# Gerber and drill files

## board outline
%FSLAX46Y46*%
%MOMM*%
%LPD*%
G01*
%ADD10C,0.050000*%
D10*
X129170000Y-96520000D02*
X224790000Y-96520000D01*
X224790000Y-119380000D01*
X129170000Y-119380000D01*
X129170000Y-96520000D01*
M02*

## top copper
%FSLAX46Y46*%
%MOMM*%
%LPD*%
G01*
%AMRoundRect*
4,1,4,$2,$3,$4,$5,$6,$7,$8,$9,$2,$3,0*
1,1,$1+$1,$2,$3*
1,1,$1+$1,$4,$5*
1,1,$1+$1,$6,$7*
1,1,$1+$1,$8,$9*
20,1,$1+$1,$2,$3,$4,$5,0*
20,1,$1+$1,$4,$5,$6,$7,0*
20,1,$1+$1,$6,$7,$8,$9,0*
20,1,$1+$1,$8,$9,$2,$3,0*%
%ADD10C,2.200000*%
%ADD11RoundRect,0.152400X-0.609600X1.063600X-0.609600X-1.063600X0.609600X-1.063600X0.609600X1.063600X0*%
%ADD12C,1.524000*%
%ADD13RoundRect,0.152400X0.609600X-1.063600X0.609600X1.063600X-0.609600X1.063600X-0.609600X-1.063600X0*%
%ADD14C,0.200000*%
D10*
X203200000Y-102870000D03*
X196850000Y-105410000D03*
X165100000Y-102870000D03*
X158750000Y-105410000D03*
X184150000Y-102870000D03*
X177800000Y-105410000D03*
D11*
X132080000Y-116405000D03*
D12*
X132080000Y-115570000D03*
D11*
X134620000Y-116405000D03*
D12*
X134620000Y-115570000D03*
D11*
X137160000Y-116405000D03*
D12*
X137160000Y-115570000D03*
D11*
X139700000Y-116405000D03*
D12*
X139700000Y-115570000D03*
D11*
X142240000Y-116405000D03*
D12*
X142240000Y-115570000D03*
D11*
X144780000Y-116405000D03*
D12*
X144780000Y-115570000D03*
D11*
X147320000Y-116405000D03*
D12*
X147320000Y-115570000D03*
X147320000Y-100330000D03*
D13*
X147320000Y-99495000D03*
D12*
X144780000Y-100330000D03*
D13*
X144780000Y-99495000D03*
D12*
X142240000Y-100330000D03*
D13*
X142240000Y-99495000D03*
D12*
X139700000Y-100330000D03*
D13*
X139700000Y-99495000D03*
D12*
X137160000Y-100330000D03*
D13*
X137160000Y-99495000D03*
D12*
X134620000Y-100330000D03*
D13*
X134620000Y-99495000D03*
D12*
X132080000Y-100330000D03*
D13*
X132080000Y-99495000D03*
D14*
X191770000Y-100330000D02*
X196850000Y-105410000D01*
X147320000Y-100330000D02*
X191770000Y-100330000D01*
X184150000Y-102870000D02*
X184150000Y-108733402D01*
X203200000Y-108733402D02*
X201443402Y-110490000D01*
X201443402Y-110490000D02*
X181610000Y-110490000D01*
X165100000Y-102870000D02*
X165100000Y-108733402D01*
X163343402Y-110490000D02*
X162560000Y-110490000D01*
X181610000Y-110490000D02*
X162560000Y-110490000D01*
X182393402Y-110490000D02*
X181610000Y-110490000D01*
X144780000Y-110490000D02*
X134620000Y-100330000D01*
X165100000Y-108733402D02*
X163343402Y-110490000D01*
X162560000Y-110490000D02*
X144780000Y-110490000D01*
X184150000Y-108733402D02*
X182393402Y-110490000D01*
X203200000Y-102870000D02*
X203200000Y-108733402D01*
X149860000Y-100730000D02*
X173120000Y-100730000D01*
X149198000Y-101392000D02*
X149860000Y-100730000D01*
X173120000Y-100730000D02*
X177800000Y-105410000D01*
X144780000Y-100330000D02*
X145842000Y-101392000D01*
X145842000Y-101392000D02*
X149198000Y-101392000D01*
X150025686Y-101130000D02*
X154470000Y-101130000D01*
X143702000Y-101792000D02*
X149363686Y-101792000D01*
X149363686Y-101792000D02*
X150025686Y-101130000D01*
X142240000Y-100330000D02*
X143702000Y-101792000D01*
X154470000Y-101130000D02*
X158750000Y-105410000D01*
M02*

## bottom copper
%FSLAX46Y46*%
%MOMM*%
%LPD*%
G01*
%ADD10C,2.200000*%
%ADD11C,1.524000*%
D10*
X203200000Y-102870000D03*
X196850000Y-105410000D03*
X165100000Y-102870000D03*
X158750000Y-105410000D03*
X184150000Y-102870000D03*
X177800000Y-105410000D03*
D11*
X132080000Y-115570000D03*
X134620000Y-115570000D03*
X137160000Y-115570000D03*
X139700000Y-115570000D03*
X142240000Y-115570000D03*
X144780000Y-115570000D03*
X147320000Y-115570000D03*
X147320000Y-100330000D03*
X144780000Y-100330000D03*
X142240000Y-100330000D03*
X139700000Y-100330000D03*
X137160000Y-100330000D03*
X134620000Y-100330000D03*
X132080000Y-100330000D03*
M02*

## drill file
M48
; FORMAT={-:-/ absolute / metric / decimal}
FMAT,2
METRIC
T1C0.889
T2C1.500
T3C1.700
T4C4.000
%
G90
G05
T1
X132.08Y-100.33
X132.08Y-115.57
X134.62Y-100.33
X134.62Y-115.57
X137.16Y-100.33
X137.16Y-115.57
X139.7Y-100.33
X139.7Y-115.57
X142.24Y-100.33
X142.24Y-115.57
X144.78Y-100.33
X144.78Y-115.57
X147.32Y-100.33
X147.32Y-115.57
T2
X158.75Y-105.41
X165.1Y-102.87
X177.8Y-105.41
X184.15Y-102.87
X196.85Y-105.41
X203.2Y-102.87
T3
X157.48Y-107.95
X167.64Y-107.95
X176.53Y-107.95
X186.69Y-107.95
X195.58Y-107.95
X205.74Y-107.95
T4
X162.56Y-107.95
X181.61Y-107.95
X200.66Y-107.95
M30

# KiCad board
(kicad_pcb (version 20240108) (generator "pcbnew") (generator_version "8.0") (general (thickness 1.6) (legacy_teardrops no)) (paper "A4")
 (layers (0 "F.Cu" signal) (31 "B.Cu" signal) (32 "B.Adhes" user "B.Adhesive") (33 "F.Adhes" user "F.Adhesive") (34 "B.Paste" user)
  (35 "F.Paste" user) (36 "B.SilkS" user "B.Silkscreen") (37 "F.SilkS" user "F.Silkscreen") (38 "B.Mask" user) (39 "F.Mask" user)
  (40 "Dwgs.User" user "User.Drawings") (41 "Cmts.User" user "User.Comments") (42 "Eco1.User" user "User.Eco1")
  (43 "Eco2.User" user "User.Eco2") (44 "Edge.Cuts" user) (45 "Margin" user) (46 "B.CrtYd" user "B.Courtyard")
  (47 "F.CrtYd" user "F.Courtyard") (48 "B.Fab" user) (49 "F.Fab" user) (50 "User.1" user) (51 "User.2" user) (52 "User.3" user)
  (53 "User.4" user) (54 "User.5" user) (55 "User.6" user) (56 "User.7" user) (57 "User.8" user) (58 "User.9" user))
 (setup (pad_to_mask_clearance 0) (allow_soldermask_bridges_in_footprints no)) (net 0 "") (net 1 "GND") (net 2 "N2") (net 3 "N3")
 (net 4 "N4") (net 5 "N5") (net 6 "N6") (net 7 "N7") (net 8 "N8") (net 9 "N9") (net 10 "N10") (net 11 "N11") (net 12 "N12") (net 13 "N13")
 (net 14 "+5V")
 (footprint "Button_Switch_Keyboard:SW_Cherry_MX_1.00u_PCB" (layer "F.Cu") (at 203.2 102.87)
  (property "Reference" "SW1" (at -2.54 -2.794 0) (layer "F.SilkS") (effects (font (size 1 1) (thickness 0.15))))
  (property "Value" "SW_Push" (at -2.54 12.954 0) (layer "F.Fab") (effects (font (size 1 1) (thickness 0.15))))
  (pad "" np_thru_hole circle (at -7.62 5.08) (size 1.7 1.7) (drill 1.7) (layers "*.Cu" "*.Mask"))
  (pad "" np_thru_hole circle (at -2.54 5.08) (size 4 4) (drill 4) (layers "*.Cu" "*.Mask"))
  (pad "" np_thru_hole circle (at 2.54 5.08) (size 1.7 1.7) (drill 1.7) (layers "*.Cu" "*.Mask"))
  (pad "1" thru_hole circle (at 0 0) (size 2.2 2.2) (drill 1.5) (layers "*.Cu" "*.Mask") (remove_unused_layers no) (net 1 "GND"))
  (pad "2" thru_hole circle (at -6.35 2.54) (size 2.2 2.2) (drill 1.5) (layers "*.Cu" "*.Mask") (remove_unused_layers no) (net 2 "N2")))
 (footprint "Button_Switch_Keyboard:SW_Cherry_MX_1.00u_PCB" (layer "F.Cu") (at 165.1 102.87)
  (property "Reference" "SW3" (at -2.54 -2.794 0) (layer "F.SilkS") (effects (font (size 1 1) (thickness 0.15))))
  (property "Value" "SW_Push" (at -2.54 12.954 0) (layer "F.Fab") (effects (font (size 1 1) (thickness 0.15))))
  (pad "" np_thru_hole circle (at -7.62 5.08) (size 1.7 1.7) (drill 1.7) (layers "*.Cu" "*.Mask"))
  (pad "" np_thru_hole circle (at -2.54 5.08) (size 4 4) (drill 4) (layers "*.Cu" "*.Mask"))
  (pad "" np_thru_hole circle (at 2.54 5.08) (size 1.7 1.7) (drill 1.7) (layers "*.Cu" "*.Mask"))
  (pad "1" thru_hole circle (at 0 0) (size 2.2 2.2) (drill 1.5) (layers "*.Cu" "*.Mask") (remove_unused_layers no) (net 1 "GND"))
  (pad "2" thru_hole circle (at -6.35 2.54) (size 2.2 2.2) (drill 1.5) (layers "*.Cu" "*.Mask") (remove_unused_layers no) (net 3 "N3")))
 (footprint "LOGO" (layer "F.Cu") (at 214.63 100.33)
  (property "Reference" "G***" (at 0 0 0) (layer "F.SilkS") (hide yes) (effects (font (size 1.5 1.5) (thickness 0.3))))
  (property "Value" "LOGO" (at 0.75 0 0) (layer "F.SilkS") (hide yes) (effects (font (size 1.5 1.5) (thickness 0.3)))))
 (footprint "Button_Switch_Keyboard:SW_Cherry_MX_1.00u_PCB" (layer "F.Cu") (at 184.15 102.87)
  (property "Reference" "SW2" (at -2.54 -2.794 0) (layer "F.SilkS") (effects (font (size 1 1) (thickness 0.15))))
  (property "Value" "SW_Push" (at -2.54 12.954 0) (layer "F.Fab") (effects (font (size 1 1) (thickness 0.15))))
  (pad "" np_thru_hole circle (at -7.62 5.08) (size 1.7 1.7) (drill 1.7) (layers "*.Cu" "*.Mask"))
  (pad "" np_thru_hole circle (at -2.54 5.08) (size 4 4) (drill 4) (layers "*.Cu" "*.Mask"))
  (pad "" np_thru_hole circle (at 2.54 5.08) (size 1.7 1.7) (drill 1.7) (layers "*.Cu" "*.Mask"))
  (pad "1" thru_hole circle (at 0 0) (size 2.2 2.2) (drill 1.5) (layers "*.Cu" "*.Mask") (remove_unused_layers no) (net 1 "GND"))
  (pad "2" thru_hole circle (at -6.35 2.54) (size 2.2 2.2) (drill 1.5) (layers "*.Cu" "*.Mask") (remove_unused_layers no) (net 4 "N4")))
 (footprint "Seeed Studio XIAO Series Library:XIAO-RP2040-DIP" (layer "F.Cu") (at 139.7 107.95 90)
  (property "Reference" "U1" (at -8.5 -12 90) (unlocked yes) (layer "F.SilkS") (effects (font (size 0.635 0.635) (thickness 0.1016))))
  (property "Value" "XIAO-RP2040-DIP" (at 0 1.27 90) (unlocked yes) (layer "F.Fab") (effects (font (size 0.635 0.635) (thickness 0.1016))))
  (pad "1" smd roundrect (at -8.455 -7.62 270) (size 2.432 1.524) (layers "F.Cu" "F.Mask") (roundrect_rratio 0.1) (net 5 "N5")
   (thermal_bridge_angle 45))
  (pad "1" thru_hole circle (at -7.62 -7.62 270) (size 1.524 1.524) (drill 0.889) (layers "*.Cu" "*.Mask") (remove_unused_layers no)
   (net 5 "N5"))
  (pad "2" smd roundrect (at -8.455 -5.08 270) (size 2.432 1.524) (layers "F.Cu" "F.Mask") (roundrect_rratio 0.1) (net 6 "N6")
   (thermal_bridge_angle 45))
  (pad "2" thru_hole circle (at -7.62 -5.08 270) (size 1.524 1.524) (drill 0.889) (layers "*.Cu" "*.Mask") (remove_unused_layers no)
   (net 6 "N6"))
  (pad "3" smd roundrect (at -8.455 -2.54 270) (size 2.432 1.524) (layers "F.Cu" "F.Mask") (roundrect_rratio 0.1) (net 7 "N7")
   (thermal_bridge_angle 45))
  (pad "3" thru_hole circle (at -7.62 -2.54 270) (size 1.524 1.524) (drill 0.889) (layers "*.Cu" "*.Mask") (remove_unused_layers no)
   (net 7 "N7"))
  (pad "4" smd roundrect (at -8.455 0 270) (size 2.432 1.524) (layers "F.Cu" "F.Mask") (roundrect_rratio 0.1) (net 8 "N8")
   (thermal_bridge_angle 45))
  (pad "4" thru_hole circle (at -7.62 0 270) (size 1.524 1.524) (drill 0.889) (layers "*.Cu" "*.Mask") (remove_unused_layers no)
   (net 8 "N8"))
  (pad "5" smd roundrect (at -8.455 2.54 270) (size 2.432 1.524) (layers "F.Cu" "F.Mask") (roundrect_rratio 0.1) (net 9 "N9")
   (thermal_bridge_angle 45))
  (pad "5" thru_hole circle (at -7.62 2.54 270) (size 1.524 1.524) (drill 0.889) (layers "*.Cu" "*.Mask") (remove_unused_layers no)
   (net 9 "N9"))
  (pad "6" smd roundrect (at -8.455 5.08 270) (size 2.432 1.524) (layers "F.Cu" "F.Mask") (roundrect_rratio 0.1) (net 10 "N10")
   (thermal_bridge_angle 45))
  (pad "6" thru_hole circle (at -7.62 5.08 270) (size 1.524 1.524) (drill 0.889) (layers "*.Cu" "*.Mask") (remove_unused_layers no)
   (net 10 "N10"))
  (pad "7" smd roundrect (at -8.455 7.62 270) (size 2.432 1.524) (layers "F.Cu" "F.Mask") (roundrect_rratio 0.1) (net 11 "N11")
   (thermal_bridge_angle 45))
  (pad "7" thru_hole circle (at -7.62 7.62 270) (size 1.524 1.524) (drill 0.889) (layers "*.Cu" "*.Mask") (remove_unused_layers no)
   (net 11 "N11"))
  (pad "8" thru_hole circle (at 7.62 7.62 90) (size 1.524 1.524) (drill 0.889) (layers "*.Cu" "*.Mask") (remove_unused_layers no)
   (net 2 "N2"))
  (pad "8" smd roundrect (at 8.455 7.62 90) (size 2.432 1.524) (layers "F.Cu" "F.Mask") (roundrect_rratio 0.1) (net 2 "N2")
   (thermal_bridge_angle 45))
  (pad "9" thru_hole circle (at 7.62 5.08 90) (size 1.524 1.524) (drill 0.889) (layers "*.Cu" "*.Mask") (remove_unused_layers no)
   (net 4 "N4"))
  (pad "9" smd roundrect (at 8.455 5.08 90) (size 2.432 1.524) (layers "F.Cu" "F.Mask") (roundrect_rratio 0.1) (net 4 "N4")
   (thermal_bridge_angle 45))
  (pad "10" thru_hole circle (at 7.62 2.54 90) (size 1.524 1.524) (drill 0.889) (layers "*.Cu" "*.Mask") (remove_unused_layers no)
   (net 3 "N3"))
  (pad "10" smd roundrect (at 8.455 2.54 90) (size 2.432 1.524) (layers "F.Cu" "F.Mask") (roundrect_rratio 0.1) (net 3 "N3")
   (thermal_bridge_angle 45))
  (pad "11" thru_hole circle (at 7.62 0 90) (size 1.524 1.524) (drill 0.889) (layers "*.Cu" "*.Mask") (remove_unused_layers no)
   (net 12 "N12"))
  (pad "11" smd roundrect (at 8.455 0 90) (size 2.432 1.524) (layers "F.Cu" "F.Mask") (roundrect_rratio 0.1) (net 12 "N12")
   (thermal_bridge_angle 45))
  (pad "12" thru_hole circle (at 7.62 -2.54 90) (size 1.524 1.524) (drill 0.889) (layers "*.Cu" "*.Mask") (remove_unused_layers no)
   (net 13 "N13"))
  (pad "12" smd roundrect (at 8.455 -2.54 90) (size 2.432 1.524) (layers "F.Cu" "F.Mask") (roundrect_rratio 0.1) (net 13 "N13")
   (thermal_bridge_angle 45))
  (pad "13" thru_hole circle (at 7.62 -5.08 90) (size 1.524 1.524) (drill 0.889) (layers "*.Cu" "*.Mask") (remove_unused_layers no)
   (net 1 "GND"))
  (pad "13" smd roundrect (at 8.455 -5.08 90) (size 2.432 1.524) (layers "F.Cu" "F.Mask") (roundrect_rratio 0.1) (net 1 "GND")
   (thermal_bridge_angle 45))
  (pad "14" thru_hole circle (at 7.62 -7.62 90) (size 1.524 1.524) (drill 0.889) (layers "*.Cu" "*.Mask") (remove_unused_layers no)
   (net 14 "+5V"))
  (pad "14" smd roundrect (at 8.455 -7.62 90) (size 2.432 1.524) (layers "F.Cu" "F.Mask") (roundrect_rratio 0.1) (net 14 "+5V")
   (thermal_bridge_angle 45)))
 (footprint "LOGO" (layer "F.Cu") (at 217.239441 111.329438)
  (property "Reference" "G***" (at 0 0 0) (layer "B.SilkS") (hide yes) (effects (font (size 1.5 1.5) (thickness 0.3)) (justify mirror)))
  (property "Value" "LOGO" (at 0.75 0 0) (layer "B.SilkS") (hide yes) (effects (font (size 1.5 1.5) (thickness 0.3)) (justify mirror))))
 (gr_rect (start 129.17 96.52) (end 224.79 119.38) (stroke (width 0.05) (type default)) (fill none) (layer "Edge.Cuts"))
 (segment (start 191.77 100.33) (end 196.85 105.41) (width 0.2) (layer "F.Cu") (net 2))
 (segment (start 147.32 100.33) (end 191.77 100.33) (width 0.2) (layer "F.Cu") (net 2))
 (segment (start 184.15 102.87) (end 184.15 108.733402) (width 0.2) (layer "F.Cu") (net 1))
 (segment (start 203.2 108.733402) (end 201.443402 110.49) (width 0.2) (layer "F.Cu") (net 1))
 (segment (start 201.443402 110.49) (end 181.61 110.49) (width 0.2) (layer "F.Cu") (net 1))
 (segment (start 165.1 102.87) (end 165.1 108.733402) (width 0.2) (layer "F.Cu") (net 1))
 (segment (start 163.343402 110.49) (end 162.56 110.49) (width 0.2) (layer "F.Cu") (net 1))
 (segment (start 181.61 110.49) (end 162.56 110.49) (width 0.2) (layer "F.Cu") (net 1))
 (segment (start 182.393402 110.49) (end 181.61 110.49) (width 0.2) (layer "F.Cu") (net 1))
 (segment (start 144.78 110.49) (end 134.62 100.33) (width 0.2) (layer "F.Cu") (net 1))
 (segment (start 165.1 108.733402) (end 163.343402 110.49) (width 0.2) (layer "F.Cu") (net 1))
 (segment (start 162.56 110.49) (end 144.78 110.49) (width 0.2) (layer "F.Cu") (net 1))
 (segment (start 184.15 108.733402) (end 182.393402 110.49) (width 0.2) (layer "F.Cu") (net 1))
 (segment (start 203.2 102.87) (end 203.2 108.733402) (width 0.2) (layer "F.Cu") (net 1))
 (segment (start 149.86 100.73) (end 173.12 100.73) (width 0.2) (layer "F.Cu") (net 4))
 (segment (start 149.198 101.392) (end 149.86 100.73) (width 0.2) (layer "F.Cu") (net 4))
 (segment (start 173.12 100.73) (end 177.8 105.41) (width 0.2) (layer "F.Cu") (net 4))
 (segment (start 144.78 100.33) (end 145.842 101.392) (width 0.2) (layer "F.Cu") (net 4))
 (segment (start 145.842 101.392) (end 149.198 101.392) (width 0.2) (layer "F.Cu") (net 4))
 (segment (start 150.025686 101.13) (end 154.47 101.13) (width 0.2) (layer "F.Cu") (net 3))
 (segment (start 143.702 101.792) (end 149.363686 101.792) (width 0.2) (layer "F.Cu") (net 3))
 (segment (start 149.363686 101.792) (end 150.025686 101.13) (width 0.2) (layer "F.Cu") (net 3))
 (segment (start 142.24 100.33) (end 143.702 101.792) (width 0.2) (layer "F.Cu") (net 3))
 (segment (start 154.47 101.13) (end 158.75 105.41) (width 0.2) (layer "F.Cu") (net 3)))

